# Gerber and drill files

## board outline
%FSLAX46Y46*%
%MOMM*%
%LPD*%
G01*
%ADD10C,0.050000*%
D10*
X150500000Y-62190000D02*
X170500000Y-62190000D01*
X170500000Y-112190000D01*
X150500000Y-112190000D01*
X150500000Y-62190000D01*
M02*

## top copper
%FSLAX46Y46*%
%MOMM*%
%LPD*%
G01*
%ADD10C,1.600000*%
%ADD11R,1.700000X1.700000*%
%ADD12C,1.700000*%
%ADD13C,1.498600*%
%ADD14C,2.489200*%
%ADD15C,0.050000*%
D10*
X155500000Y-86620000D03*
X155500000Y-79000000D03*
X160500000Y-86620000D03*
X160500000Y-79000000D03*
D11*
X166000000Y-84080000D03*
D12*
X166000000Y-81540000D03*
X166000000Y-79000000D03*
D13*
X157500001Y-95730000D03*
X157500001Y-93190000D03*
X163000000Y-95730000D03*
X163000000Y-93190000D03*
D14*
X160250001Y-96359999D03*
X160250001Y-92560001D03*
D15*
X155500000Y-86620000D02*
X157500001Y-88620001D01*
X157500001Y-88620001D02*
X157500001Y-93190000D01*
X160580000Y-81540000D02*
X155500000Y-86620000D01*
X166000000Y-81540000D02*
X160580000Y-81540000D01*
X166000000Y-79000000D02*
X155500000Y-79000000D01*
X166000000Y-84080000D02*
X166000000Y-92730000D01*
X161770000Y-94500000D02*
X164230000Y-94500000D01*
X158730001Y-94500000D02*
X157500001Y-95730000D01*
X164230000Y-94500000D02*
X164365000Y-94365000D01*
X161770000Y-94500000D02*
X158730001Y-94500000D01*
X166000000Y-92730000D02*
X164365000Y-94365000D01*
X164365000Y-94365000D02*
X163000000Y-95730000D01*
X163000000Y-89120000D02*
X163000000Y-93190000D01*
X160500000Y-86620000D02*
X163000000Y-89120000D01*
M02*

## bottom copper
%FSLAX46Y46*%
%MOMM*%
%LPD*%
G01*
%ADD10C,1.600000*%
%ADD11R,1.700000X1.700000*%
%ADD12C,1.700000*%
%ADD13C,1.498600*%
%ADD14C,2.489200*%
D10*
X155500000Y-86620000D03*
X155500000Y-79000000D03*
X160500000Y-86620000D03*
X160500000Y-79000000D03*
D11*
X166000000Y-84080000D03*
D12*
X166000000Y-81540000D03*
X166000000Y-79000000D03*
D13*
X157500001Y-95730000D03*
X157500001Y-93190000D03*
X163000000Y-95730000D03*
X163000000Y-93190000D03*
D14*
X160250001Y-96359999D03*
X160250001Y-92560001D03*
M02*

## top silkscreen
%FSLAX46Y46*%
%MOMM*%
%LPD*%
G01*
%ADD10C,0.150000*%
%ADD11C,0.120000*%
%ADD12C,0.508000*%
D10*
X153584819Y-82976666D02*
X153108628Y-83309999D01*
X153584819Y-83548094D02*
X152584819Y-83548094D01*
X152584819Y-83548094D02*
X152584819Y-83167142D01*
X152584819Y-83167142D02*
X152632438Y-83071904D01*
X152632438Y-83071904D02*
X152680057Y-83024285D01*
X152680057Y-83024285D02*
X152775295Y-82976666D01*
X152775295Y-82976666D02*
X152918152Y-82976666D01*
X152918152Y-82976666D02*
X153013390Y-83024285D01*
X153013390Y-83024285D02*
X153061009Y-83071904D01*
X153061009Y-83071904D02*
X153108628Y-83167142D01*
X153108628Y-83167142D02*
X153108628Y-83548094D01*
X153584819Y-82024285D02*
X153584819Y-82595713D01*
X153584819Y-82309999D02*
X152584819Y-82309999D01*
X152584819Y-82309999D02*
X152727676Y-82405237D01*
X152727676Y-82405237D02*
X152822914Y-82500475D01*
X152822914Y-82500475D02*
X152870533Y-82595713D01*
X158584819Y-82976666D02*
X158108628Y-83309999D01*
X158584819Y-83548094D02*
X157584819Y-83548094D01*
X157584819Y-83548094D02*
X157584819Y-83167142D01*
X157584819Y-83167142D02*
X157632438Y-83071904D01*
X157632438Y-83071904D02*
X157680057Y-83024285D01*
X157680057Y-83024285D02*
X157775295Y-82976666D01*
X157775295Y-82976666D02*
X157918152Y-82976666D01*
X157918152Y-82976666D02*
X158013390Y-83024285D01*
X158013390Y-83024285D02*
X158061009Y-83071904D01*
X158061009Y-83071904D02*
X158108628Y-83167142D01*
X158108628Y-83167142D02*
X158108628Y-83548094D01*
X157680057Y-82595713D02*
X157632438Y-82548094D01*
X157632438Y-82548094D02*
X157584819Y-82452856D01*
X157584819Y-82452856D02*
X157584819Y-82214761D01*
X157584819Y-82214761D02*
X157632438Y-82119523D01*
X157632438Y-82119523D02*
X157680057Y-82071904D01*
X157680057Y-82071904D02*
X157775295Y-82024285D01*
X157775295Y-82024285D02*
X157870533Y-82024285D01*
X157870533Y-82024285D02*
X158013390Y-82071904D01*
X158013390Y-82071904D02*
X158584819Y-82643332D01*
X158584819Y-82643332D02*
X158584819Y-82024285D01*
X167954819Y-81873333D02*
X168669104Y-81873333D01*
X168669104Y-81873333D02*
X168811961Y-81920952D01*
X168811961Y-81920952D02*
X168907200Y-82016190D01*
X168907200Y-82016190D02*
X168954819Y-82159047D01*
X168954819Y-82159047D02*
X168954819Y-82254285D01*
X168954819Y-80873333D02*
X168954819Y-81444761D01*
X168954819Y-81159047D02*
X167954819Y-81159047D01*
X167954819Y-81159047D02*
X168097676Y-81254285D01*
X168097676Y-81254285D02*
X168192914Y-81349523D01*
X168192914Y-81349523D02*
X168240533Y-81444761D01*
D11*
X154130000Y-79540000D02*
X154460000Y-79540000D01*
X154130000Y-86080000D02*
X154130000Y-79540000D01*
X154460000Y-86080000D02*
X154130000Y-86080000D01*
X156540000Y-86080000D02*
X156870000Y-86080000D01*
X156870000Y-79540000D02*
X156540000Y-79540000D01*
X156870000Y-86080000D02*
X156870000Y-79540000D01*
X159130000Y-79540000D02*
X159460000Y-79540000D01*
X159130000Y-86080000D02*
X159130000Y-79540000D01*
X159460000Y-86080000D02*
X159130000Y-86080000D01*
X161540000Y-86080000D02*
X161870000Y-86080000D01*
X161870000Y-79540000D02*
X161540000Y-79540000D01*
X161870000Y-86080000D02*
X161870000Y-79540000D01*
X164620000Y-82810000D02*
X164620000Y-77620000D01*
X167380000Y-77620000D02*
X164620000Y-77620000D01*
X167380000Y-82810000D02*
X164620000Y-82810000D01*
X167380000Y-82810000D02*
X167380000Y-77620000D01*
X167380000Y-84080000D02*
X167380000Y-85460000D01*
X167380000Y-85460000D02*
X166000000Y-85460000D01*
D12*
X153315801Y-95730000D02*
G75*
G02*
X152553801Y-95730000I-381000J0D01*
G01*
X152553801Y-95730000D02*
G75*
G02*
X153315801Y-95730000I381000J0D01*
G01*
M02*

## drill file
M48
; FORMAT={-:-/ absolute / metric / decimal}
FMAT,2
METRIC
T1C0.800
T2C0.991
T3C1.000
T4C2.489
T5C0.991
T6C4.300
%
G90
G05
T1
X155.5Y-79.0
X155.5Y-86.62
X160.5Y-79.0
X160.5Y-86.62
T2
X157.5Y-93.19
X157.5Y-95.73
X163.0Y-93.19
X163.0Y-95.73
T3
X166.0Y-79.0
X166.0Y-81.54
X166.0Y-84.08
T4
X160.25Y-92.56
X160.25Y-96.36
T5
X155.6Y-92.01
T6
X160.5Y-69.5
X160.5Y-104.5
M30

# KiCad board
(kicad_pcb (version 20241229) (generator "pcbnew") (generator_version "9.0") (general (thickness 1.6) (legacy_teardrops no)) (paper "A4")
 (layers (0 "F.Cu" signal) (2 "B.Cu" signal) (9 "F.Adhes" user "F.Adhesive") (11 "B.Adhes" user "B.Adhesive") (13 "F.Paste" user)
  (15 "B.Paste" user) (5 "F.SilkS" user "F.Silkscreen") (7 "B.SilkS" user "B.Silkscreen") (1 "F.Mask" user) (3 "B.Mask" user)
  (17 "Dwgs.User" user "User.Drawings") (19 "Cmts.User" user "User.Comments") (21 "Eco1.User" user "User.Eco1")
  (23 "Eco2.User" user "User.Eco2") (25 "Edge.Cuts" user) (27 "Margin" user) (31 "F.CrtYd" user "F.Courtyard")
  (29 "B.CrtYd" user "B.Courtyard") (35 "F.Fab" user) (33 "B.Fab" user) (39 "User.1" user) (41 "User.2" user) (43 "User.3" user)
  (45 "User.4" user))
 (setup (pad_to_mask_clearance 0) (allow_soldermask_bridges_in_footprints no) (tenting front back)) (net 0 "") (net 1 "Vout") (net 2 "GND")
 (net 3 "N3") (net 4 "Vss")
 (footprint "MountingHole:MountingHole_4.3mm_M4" (layer "F.Cu") (at 160.5 69.5)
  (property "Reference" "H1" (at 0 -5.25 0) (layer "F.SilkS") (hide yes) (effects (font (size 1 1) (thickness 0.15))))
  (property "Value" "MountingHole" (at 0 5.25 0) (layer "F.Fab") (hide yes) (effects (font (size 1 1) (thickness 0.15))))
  (pad "" np_thru_hole circle (at 0 0) (size 4.3 4.3) (drill 4.3) (layers "*.Cu" "*.Mask")))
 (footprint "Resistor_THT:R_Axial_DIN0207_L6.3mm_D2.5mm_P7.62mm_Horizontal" (layer "F.Cu") (at 155.5 86.62 90)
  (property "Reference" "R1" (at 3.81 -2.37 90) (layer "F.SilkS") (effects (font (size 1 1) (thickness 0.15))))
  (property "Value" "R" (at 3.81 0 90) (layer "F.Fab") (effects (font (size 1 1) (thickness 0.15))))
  (fp_line (start 7.08 -1.37) (end 7.08 -1.04) (stroke (width 0.12) (type solid)) (layer "F.SilkS"))
  (fp_line (start 0.54 -1.37) (end 7.08 -1.37) (stroke (width 0.12) (type solid)) (layer "F.SilkS"))
  (fp_line (start 0.54 -1.04) (end 0.54 -1.37) (stroke (width 0.12) (type solid)) (layer "F.SilkS"))
  (fp_line (start 0.54 1.04) (end 0.54 1.37) (stroke (width 0.12) (type solid)) (layer "F.SilkS"))
  (fp_line (start 7.08 1.37) (end 7.08 1.04) (stroke (width 0.12) (type solid)) (layer "F.SilkS"))
  (fp_line (start 0.54 1.37) (end 7.08 1.37) (stroke (width 0.12) (type solid)) (layer "F.SilkS"))
  (pad "1" thru_hole circle (at 0 0 90) (size 1.6 1.6) (drill 0.8) (layers "*.Cu" "*.Mask") (remove_unused_layers no) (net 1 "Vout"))
  (pad "2" thru_hole circle (at 7.62 0 90) (size 1.6 1.6) (drill 0.8) (layers "*.Cu" "*.Mask") (remove_unused_layers no) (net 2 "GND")))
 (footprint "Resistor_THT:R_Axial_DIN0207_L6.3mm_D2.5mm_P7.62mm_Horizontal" (layer "F.Cu") (at 160.5 86.62 90)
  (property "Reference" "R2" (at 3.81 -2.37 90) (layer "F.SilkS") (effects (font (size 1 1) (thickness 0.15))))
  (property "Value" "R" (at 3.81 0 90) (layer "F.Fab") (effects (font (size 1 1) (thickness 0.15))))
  (fp_line (start 7.08 -1.37) (end 7.08 -1.04) (stroke (width 0.12) (type solid)) (layer "F.SilkS"))
  (fp_line (start 0.54 -1.37) (end 7.08 -1.37) (stroke (width 0.12) (type solid)) (layer "F.SilkS"))
  (fp_line (start 0.54 -1.04) (end 0.54 -1.37) (stroke (width 0.12) (type solid)) (layer "F.SilkS"))
  (fp_line (start 0.54 1.04) (end 0.54 1.37) (stroke (width 0.12) (type solid)) (layer "F.SilkS"))
  (fp_line (start 7.08 1.37) (end 7.08 1.04) (stroke (width 0.12) (type solid)) (layer "F.SilkS"))
  (fp_line (start 0.54 1.37) (end 7.08 1.37) (stroke (width 0.12) (type solid)) (layer "F.SilkS"))
  (pad "1" thru_hole circle (at 0 0 90) (size 1.6 1.6) (drill 0.8) (layers "*.Cu" "*.Mask") (remove_unused_layers no) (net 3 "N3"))
  (pad "2" thru_hole circle (at 7.62 0 90) (size 1.6 1.6) (drill 0.8) (layers "*.Cu" "*.Mask") (remove_unused_layers no) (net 2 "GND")))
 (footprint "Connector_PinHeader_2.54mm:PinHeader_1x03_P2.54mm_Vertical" (layer "F.Cu") (at 166 84.08 180)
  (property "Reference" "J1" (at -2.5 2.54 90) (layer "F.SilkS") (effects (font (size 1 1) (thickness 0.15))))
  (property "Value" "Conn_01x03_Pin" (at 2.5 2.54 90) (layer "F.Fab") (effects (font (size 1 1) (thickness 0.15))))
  (fp_line (start 1.38 1.27) (end 1.38 6.46) (stroke (width 0.12) (type solid)) (layer "F.SilkS"))
  (fp_line (start -1.38 6.46) (end 1.38 6.46) (stroke (width 0.12) (type solid)) (layer "F.SilkS"))
  (fp_line (start -1.38 1.27) (end 1.38 1.27) (stroke (width 0.12) (type solid)) (layer "F.SilkS"))
  (fp_line (start -1.38 1.27) (end -1.38 6.46) (stroke (width 0.12) (type solid)) (layer "F.SilkS"))
  (fp_line (start -1.38 0) (end -1.38 -1.38) (stroke (width 0.12) (type solid)) (layer "F.SilkS"))
  (fp_line (start -1.38 -1.38) (end 0 -1.38) (stroke (width 0.12) (type solid)) (layer "F.SilkS"))
  (pad "1" thru_hole rect (at 0 0 180) (size 1.7 1.7) (drill 1) (layers "*.Cu" "*.Mask") (remove_unused_layers no) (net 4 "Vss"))
  (pad "2" thru_hole circle (at 0 2.54 180) (size 1.7 1.7) (drill 1) (layers "*.Cu" "*.Mask") (remove_unused_layers no) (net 1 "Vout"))
  (pad "3" thru_hole circle (at 0 5.08 180) (size 1.7 1.7) (drill 1) (layers "*.Cu" "*.Mask") (remove_unused_layers no) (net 2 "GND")))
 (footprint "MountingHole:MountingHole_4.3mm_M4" (layer "F.Cu") (at 160.5 104.5)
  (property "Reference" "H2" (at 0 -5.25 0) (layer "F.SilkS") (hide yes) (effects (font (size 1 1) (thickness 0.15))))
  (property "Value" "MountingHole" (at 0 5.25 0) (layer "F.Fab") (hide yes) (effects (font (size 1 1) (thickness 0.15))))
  (pad "" np_thru_hole circle (at 0 0) (size 4.3 4.3) (drill 4.3) (layers "*.Cu" "*.Mask")))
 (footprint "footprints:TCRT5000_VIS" (layer "B.Cu") (at 157.500001 95.73)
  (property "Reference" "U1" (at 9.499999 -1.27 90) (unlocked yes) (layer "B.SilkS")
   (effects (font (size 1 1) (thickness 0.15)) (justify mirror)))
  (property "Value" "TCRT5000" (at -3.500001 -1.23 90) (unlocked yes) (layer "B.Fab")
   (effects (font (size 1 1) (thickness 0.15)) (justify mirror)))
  (fp_circle (center -4.5652 0) (end -4.1842 0) (stroke (width 0.508) (type solid)) (fill no) (layer "F.SilkS"))
  (pad "" np_thru_hole circle (at -1.900001 -3.72) (size 0.9906 0.9906) (drill 0.9906) (layers "*.Cu" "*.Mask"))
  (pad "1" thru_hole circle (at 0 0) (size 1.4986 1.4986) (drill 0.9906) (layers "*.Cu" "*.Mask") (remove_unused_layers no) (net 4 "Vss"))
  (pad "2" thru_hole circle (at 0 -2.54) (size 1.4986 1.4986) (drill 0.9906) (layers "*.Cu" "*.Mask") (remove_unused_layers no)
   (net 1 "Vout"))
  (pad "3" thru_hole circle (at 5.499999 0) (size 1.4986 1.4986) (drill 0.9906) (layers "*.Cu" "*.Mask") (remove_unused_layers no)
   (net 4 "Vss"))
  (pad "4" thru_hole circle (at 5.499999 -2.54) (size 1.4986 1.4986) (drill 0.9906) (layers "*.Cu" "*.Mask") (remove_unused_layers no)
   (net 3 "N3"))
  (pad "5" thru_hole circle (at 2.75 0.629999) (size 2.4892 2.4892) (drill 2.4892) (layers "*.Cu" "*.Mask") (remove_unused_layers no))
  (pad "6" thru_hole circle (at 2.75 -3.169999) (size 2.4892 2.4892) (drill 2.4892) (layers "*.Cu" "*.Mask") (remove_unused_layers no)))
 (gr_rect (start 150.5 62.19) (end 170.5 112.19) (stroke (width 0.05) (type default)) (fill no) (layer "Edge.Cuts"))
 (segment (start 155.5 86.62) (end 157.500001 88.620001) (width 0.05) (layer "F.Cu") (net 1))
 (segment (start 157.500001 88.620001) (end 157.500001 93.19) (width 0.05) (layer "F.Cu") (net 1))
 (segment (start 160.58 81.54) (end 155.5 86.62) (width 0.05) (layer "F.Cu") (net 1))
 (segment (start 166 81.54) (end 160.58 81.54) (width 0.05) (layer "F.Cu") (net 1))
 (segment (start 166 79) (end 155.5 79) (width 0.05) (layer "F.Cu") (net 2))
 (segment (start 166 84.08) (end 166 92.73) (width 0.05) (layer "F.Cu") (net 4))
 (segment (start 161.77 94.5) (end 164.23 94.5) (width 0.05) (layer "F.Cu") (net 4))
 (segment (start 158.730001 94.5) (end 157.500001 95.73) (width 0.05) (layer "F.Cu") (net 4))
 (segment (start 164.23 94.5) (end 164.365 94.365) (width 0.05) (layer "F.Cu") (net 4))
 (segment (start 161.77 94.5) (end 158.730001 94.5) (width 0.05) (layer "F.Cu") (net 4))
 (segment (start 166 92.73) (end 164.365 94.365) (width 0.05) (layer "F.Cu") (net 4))
 (segment (start 164.365 94.365) (end 163 95.73) (width 0.05) (layer "F.Cu") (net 4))
 (segment (start 163 89.12) (end 163 93.19) (width 0.05) (layer "F.Cu") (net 3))
 (segment (start 160.5 86.62) (end 163 89.12) (width 0.05) (layer "F.Cu") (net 3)))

